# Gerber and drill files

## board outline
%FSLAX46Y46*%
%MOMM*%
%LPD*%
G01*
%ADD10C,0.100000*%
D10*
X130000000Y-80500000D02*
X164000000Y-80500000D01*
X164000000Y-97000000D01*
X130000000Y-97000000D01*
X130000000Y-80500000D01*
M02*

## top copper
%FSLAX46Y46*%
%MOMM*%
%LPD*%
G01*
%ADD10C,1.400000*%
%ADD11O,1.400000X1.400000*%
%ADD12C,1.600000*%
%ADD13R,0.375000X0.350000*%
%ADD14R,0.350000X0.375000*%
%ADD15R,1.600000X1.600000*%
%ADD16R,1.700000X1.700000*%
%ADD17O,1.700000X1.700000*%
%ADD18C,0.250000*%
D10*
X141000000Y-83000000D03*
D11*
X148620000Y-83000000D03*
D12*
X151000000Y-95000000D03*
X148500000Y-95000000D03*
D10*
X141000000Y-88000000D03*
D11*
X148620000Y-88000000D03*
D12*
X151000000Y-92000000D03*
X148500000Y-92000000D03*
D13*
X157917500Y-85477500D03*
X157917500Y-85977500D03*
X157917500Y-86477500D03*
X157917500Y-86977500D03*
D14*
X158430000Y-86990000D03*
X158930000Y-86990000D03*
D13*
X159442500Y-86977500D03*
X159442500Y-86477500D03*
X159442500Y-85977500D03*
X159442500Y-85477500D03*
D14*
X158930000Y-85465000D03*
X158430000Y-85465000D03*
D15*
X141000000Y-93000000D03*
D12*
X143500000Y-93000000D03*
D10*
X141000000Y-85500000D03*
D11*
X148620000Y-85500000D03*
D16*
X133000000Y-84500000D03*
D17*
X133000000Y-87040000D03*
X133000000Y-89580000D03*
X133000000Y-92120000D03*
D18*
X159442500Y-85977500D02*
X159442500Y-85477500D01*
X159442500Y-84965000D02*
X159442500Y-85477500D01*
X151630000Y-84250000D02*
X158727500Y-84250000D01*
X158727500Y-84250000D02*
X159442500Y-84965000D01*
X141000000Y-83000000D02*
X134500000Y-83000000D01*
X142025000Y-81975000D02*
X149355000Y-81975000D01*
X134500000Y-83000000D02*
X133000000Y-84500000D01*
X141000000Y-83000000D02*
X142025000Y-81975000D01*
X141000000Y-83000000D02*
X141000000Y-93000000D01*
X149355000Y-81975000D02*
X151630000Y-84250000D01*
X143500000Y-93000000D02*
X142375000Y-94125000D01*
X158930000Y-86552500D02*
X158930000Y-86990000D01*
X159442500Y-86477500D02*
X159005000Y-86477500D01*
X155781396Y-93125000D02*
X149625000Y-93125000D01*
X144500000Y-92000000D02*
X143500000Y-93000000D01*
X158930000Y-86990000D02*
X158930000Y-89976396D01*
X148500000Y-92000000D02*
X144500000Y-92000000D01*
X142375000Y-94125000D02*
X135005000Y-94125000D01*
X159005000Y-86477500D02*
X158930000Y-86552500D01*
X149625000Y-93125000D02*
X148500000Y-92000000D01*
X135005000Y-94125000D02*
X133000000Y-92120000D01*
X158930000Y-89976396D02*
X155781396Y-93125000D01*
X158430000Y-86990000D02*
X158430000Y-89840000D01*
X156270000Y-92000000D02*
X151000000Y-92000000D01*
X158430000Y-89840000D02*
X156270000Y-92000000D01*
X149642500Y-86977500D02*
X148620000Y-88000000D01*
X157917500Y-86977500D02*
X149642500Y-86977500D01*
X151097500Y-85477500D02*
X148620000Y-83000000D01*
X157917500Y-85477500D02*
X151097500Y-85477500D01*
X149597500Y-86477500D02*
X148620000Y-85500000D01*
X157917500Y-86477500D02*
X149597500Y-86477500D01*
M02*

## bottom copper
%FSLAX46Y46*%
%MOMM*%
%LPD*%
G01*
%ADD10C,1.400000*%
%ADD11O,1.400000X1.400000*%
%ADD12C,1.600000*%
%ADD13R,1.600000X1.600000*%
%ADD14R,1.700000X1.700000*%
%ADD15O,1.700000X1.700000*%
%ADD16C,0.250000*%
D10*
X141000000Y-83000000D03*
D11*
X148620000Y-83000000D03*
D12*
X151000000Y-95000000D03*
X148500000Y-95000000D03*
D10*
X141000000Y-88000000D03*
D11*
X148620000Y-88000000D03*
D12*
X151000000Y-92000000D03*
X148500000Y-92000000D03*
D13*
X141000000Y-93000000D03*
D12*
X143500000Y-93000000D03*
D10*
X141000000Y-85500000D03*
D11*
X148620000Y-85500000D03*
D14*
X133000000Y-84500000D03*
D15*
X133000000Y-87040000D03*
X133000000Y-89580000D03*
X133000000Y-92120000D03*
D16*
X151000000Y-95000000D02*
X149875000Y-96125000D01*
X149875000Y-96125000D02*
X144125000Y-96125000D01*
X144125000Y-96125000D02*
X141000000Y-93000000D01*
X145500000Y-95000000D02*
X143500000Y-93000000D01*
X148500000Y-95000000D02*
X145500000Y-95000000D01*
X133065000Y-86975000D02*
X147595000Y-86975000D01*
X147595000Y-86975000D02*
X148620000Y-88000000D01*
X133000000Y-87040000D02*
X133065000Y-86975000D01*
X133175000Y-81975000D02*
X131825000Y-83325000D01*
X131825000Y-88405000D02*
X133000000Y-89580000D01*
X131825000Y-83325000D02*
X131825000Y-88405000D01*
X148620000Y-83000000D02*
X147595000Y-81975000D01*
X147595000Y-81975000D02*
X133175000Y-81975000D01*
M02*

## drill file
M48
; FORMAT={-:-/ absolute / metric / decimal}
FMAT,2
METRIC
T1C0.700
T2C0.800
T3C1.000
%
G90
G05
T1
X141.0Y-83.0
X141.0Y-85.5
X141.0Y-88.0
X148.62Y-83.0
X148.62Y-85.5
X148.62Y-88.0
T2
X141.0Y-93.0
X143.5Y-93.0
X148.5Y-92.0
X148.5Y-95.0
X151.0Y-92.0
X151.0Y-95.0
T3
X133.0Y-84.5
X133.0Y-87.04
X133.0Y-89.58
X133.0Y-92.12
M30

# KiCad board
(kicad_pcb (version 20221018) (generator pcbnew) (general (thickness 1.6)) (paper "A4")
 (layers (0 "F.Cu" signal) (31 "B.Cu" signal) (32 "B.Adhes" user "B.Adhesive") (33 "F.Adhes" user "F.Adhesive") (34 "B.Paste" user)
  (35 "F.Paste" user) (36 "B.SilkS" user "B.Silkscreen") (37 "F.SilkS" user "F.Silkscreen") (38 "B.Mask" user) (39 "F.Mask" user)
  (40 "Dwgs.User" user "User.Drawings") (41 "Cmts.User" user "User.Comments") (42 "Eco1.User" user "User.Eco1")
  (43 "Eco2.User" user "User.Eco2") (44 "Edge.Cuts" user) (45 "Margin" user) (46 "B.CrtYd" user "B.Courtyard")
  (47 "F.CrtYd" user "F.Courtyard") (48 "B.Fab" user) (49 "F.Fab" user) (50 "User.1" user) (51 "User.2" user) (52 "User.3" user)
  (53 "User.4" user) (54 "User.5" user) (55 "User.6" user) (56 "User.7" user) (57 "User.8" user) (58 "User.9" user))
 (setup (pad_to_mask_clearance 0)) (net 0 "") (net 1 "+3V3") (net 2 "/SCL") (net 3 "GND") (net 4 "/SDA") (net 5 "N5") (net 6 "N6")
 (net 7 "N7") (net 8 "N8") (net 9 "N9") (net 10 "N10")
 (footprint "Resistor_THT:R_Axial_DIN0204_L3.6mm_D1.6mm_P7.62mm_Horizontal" (layer "F.Cu") (at 141 83)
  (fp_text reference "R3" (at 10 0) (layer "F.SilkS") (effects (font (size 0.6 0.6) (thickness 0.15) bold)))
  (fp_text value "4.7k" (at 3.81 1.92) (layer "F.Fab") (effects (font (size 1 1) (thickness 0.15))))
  (pad "1" thru_hole circle (at 0 0) (size 1.4 1.4) (drill 0.7) (layers "*.Cu" "*.Mask") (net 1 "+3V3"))
  (pad "2" thru_hole oval (at 7.62 0) (size 1.4 1.4) (drill 0.7) (layers "*.Cu" "*.Mask") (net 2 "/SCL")))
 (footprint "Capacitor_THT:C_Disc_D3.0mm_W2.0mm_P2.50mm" (layer "F.Cu") (at 151 95 180)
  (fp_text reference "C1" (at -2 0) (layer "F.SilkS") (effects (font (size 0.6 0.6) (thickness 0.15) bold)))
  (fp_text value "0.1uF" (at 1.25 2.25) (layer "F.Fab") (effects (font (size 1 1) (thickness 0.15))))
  (pad "1" thru_hole circle (at 0 0 180) (size 1.6 1.6) (drill 0.8) (layers "*.Cu" "*.Mask") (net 1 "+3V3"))
  (pad "2" thru_hole circle (at 2.5 0 180) (size 1.6 1.6) (drill 0.8) (layers "*.Cu" "*.Mask") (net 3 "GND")))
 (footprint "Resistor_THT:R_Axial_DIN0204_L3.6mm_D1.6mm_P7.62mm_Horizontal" (layer "F.Cu") (at 141 88)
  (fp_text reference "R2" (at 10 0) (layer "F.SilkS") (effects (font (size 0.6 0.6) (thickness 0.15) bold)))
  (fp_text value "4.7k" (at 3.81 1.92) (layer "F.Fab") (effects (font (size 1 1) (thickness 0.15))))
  (pad "1" thru_hole circle (at 0 0) (size 1.4 1.4) (drill 0.7) (layers "*.Cu" "*.Mask") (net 1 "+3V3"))
  (pad "2" thru_hole oval (at 7.62 0) (size 1.4 1.4) (drill 0.7) (layers "*.Cu" "*.Mask") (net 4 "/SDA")))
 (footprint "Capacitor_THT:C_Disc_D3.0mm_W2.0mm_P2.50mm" (layer "F.Cu") (at 151 92 180)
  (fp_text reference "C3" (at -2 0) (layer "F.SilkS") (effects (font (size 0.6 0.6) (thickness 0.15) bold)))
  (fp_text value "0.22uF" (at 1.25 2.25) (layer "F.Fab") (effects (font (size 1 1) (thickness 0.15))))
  (pad "1" thru_hole circle (at 0 0 180) (size 1.6 1.6) (drill 0.8) (layers "*.Cu" "*.Mask") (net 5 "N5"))
  (pad "2" thru_hole circle (at 2.5 0 180) (size 1.6 1.6) (drill 0.8) (layers "*.Cu" "*.Mask") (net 3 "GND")))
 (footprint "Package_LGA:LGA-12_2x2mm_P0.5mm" (layer "F.Cu") (at 158.68 86.2275) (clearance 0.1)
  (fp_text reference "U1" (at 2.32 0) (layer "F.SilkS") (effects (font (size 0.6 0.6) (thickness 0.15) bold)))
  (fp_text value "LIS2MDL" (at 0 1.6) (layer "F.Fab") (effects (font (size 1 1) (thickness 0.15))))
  (pad "1" smd rect (at -0.7625 -0.75) (size 0.375 0.35) (layers "F.Cu" "F.Paste" "F.Mask") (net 2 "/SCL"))
  (pad "2" smd rect (at -0.7625 -0.25) (size 0.375 0.35) (layers "F.Cu" "F.Paste" "F.Mask") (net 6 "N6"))
  (pad "3" smd rect (at -0.7625 0.25) (size 0.375 0.35) (layers "F.Cu" "F.Paste" "F.Mask") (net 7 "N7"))
  (pad "4" smd rect (at -0.7625 0.75) (size 0.375 0.35) (layers "F.Cu" "F.Paste" "F.Mask") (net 4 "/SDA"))
  (pad "5" smd rect (at -0.25 0.7625 90) (size 0.375 0.35) (layers "F.Cu" "F.Paste" "F.Mask") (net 5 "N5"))
  (pad "6" smd rect (at 0.25 0.7625 90) (size 0.375 0.35) (layers "F.Cu" "F.Paste" "F.Mask") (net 3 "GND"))
  (pad "7" smd rect (at 0.7625 0.75) (size 0.375 0.35) (layers "F.Cu" "F.Paste" "F.Mask") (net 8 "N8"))
  (pad "8" smd rect (at 0.7625 0.25) (size 0.375 0.35) (layers "F.Cu" "F.Paste" "F.Mask") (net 3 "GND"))
  (pad "9" smd rect (at 0.7625 -0.25) (size 0.375 0.35) (layers "F.Cu" "F.Paste" "F.Mask") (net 1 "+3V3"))
  (pad "10" smd rect (at 0.7625 -0.75) (size 0.375 0.35) (layers "F.Cu" "F.Paste" "F.Mask") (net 1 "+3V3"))
  (pad "11" smd rect (at 0.25 -0.7625 90) (size 0.375 0.35) (layers "F.Cu" "F.Paste" "F.Mask") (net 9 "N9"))
  (pad "12" smd rect (at -0.25 -0.7625 90) (size 0.375 0.35) (layers "F.Cu" "F.Paste" "F.Mask") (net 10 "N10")))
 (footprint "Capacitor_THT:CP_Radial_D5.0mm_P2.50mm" (layer "F.Cu") (at 141 93)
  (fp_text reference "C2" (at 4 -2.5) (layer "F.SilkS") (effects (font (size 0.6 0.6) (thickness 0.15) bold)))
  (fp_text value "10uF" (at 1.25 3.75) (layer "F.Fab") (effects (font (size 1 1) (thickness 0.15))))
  (pad "1" thru_hole rect (at 0 0) (size 1.6 1.6) (drill 0.8) (layers "*.Cu" "*.Mask") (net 1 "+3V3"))
  (pad "2" thru_hole circle (at 2.5 0) (size 1.6 1.6) (drill 0.8) (layers "*.Cu" "*.Mask") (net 3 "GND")))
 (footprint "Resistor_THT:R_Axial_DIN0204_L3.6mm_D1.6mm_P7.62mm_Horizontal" (layer "F.Cu") (at 141 85.5)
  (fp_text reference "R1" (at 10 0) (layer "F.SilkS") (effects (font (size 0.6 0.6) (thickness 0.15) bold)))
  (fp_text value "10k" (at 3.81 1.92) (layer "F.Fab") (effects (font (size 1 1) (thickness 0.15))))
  (pad "1" thru_hole circle (at 0 0) (size 1.4 1.4) (drill 0.7) (layers "*.Cu" "*.Mask") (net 1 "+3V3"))
  (pad "2" thru_hole oval (at 7.62 0) (size 1.4 1.4) (drill 0.7) (layers "*.Cu" "*.Mask") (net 7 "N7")))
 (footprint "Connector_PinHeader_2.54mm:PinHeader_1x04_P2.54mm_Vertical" (layer "F.Cu") (at 133 84.5)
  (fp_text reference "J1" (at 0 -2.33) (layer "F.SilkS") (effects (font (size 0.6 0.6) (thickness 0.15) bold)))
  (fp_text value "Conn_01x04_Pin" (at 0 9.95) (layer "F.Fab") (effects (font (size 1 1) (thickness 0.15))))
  (pad "1" thru_hole rect (at 0 0) (size 1.7 1.7) (drill 1) (layers "*.Cu" "*.Mask") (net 1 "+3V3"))
  (pad "2" thru_hole oval (at 0 2.54) (size 1.7 1.7) (drill 1) (layers "*.Cu" "*.Mask") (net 4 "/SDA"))
  (pad "3" thru_hole oval (at 0 5.08) (size 1.7 1.7) (drill 1) (layers "*.Cu" "*.Mask") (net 2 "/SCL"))
  (pad "4" thru_hole oval (at 0 7.62) (size 1.7 1.7) (drill 1) (layers "*.Cu" "*.Mask") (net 3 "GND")))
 (gr_rect (start 130 80.5) (end 164 97) (stroke (width 0.1) (type default)) (fill none) (layer "Edge.Cuts"))
 (segment (start 159.4425 85.9775) (end 159.4425 85.4775) (width 0.25) (layer "F.Cu") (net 1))
 (segment (start 159.4425 84.965) (end 159.4425 85.4775) (width 0.25) (layer "F.Cu") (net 1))
 (segment (start 151.63 84.25) (end 158.7275 84.25) (width 0.25) (layer "F.Cu") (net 1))
 (segment (start 158.7275 84.25) (end 159.4425 84.965) (width 0.25) (layer "F.Cu") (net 1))
 (segment (start 141 83) (end 134.5 83) (width 0.25) (layer "F.Cu") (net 1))
 (segment (start 142.025 81.975) (end 149.355 81.975) (width 0.25) (layer "F.Cu") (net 1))
 (segment (start 134.5 83) (end 133 84.5) (width 0.25) (layer "F.Cu") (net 1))
 (segment (start 141 83) (end 142.025 81.975) (width 0.25) (layer "F.Cu") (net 1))
 (segment (start 141 83) (end 141 93) (width 0.25) (layer "F.Cu") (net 1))
 (segment (start 149.355 81.975) (end 151.63 84.25) (width 0.25) (layer "F.Cu") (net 1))
 (segment (start 151 95) (end 149.875 96.125) (width 0.25) (layer "B.Cu") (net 1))
 (segment (start 149.875 96.125) (end 144.125 96.125) (width 0.25) (layer "B.Cu") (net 1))
 (segment (start 144.125 96.125) (end 141 93) (width 0.25) (layer "B.Cu") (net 1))
 (segment (start 143.5 93) (end 142.375 94.125) (width 0.25) (layer "F.Cu") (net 3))
 (segment (start 158.93 86.5525) (end 158.93 86.99) (width 0.25) (layer "F.Cu") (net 3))
 (segment (start 159.4425 86.4775) (end 159.005 86.4775) (width 0.25) (layer "F.Cu") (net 3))
 (segment (start 155.781396 93.125) (end 149.625 93.125) (width 0.25) (layer "F.Cu") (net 3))
 (segment (start 144.5 92) (end 143.5 93) (width 0.25) (layer "F.Cu") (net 3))
 (segment (start 158.93 86.99) (end 158.93 89.976396) (width 0.25) (layer "F.Cu") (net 3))
 (segment (start 148.5 92) (end 144.5 92) (width 0.25) (layer "F.Cu") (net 3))
 (segment (start 142.375 94.125) (end 135.005 94.125) (width 0.25) (layer "F.Cu") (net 3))
 (segment (start 159.005 86.4775) (end 158.93 86.5525) (width 0.25) (layer "F.Cu") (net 3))
 (segment (start 149.625 93.125) (end 148.5 92) (width 0.25) (layer "F.Cu") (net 3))
 (segment (start 135.005 94.125) (end 133 92.12) (width 0.25) (layer "F.Cu") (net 3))
 (segment (start 158.93 89.976396) (end 155.781396 93.125) (width 0.25) (layer "F.Cu") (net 3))
 (segment (start 145.5 95) (end 143.5 93) (width 0.25) (layer "B.Cu") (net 3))
 (segment (start 148.5 95) (end 145.5 95) (width 0.25) (layer "B.Cu") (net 3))
 (segment (start 158.43 86.99) (end 158.43 89.84) (width 0.25) (layer "F.Cu") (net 5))
 (segment (start 156.27 92) (end 151 92) (width 0.25) (layer "F.Cu") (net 5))
 (segment (start 158.43 89.84) (end 156.27 92) (width 0.25) (layer "F.Cu") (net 5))
 (segment (start 149.6425 86.9775) (end 148.62 88) (width 0.25) (layer "F.Cu") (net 4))
 (segment (start 157.9175 86.9775) (end 149.6425 86.9775) (width 0.25) (layer "F.Cu") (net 4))
 (segment (start 133.065 86.975) (end 147.595 86.975) (width 0.25) (layer "B.Cu") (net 4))
 (segment (start 147.595 86.975) (end 148.62 88) (width 0.25) (layer "B.Cu") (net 4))
 (segment (start 133 87.04) (end 133.065 86.975) (width 0.25) (layer "B.Cu") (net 4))
 (segment (start 151.0975 85.4775) (end 148.62 83) (width 0.25) (layer "F.Cu") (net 2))
 (segment (start 157.9175 85.4775) (end 151.0975 85.4775) (width 0.25) (layer "F.Cu") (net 2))
 (segment (start 133.175 81.975) (end 131.825 83.325) (width 0.25) (layer "B.Cu") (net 2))
 (segment (start 131.825 88.405) (end 133 89.58) (width 0.25) (layer "B.Cu") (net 2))
 (segment (start 131.825 83.325) (end 131.825 88.405) (width 0.25) (layer "B.Cu") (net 2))
 (segment (start 148.62 83) (end 147.595 81.975) (width 0.25) (layer "B.Cu") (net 2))
 (segment (start 147.595 81.975) (end 133.175 81.975) (width 0.25) (layer "B.Cu") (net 2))
 (segment (start 149.5975 86.4775) (end 148.62 85.5) (width 0.25) (layer "F.Cu") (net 7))
 (segment (start 157.9175 86.4775) (end 149.5975 86.4775) (width 0.25) (layer "F.Cu") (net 7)))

